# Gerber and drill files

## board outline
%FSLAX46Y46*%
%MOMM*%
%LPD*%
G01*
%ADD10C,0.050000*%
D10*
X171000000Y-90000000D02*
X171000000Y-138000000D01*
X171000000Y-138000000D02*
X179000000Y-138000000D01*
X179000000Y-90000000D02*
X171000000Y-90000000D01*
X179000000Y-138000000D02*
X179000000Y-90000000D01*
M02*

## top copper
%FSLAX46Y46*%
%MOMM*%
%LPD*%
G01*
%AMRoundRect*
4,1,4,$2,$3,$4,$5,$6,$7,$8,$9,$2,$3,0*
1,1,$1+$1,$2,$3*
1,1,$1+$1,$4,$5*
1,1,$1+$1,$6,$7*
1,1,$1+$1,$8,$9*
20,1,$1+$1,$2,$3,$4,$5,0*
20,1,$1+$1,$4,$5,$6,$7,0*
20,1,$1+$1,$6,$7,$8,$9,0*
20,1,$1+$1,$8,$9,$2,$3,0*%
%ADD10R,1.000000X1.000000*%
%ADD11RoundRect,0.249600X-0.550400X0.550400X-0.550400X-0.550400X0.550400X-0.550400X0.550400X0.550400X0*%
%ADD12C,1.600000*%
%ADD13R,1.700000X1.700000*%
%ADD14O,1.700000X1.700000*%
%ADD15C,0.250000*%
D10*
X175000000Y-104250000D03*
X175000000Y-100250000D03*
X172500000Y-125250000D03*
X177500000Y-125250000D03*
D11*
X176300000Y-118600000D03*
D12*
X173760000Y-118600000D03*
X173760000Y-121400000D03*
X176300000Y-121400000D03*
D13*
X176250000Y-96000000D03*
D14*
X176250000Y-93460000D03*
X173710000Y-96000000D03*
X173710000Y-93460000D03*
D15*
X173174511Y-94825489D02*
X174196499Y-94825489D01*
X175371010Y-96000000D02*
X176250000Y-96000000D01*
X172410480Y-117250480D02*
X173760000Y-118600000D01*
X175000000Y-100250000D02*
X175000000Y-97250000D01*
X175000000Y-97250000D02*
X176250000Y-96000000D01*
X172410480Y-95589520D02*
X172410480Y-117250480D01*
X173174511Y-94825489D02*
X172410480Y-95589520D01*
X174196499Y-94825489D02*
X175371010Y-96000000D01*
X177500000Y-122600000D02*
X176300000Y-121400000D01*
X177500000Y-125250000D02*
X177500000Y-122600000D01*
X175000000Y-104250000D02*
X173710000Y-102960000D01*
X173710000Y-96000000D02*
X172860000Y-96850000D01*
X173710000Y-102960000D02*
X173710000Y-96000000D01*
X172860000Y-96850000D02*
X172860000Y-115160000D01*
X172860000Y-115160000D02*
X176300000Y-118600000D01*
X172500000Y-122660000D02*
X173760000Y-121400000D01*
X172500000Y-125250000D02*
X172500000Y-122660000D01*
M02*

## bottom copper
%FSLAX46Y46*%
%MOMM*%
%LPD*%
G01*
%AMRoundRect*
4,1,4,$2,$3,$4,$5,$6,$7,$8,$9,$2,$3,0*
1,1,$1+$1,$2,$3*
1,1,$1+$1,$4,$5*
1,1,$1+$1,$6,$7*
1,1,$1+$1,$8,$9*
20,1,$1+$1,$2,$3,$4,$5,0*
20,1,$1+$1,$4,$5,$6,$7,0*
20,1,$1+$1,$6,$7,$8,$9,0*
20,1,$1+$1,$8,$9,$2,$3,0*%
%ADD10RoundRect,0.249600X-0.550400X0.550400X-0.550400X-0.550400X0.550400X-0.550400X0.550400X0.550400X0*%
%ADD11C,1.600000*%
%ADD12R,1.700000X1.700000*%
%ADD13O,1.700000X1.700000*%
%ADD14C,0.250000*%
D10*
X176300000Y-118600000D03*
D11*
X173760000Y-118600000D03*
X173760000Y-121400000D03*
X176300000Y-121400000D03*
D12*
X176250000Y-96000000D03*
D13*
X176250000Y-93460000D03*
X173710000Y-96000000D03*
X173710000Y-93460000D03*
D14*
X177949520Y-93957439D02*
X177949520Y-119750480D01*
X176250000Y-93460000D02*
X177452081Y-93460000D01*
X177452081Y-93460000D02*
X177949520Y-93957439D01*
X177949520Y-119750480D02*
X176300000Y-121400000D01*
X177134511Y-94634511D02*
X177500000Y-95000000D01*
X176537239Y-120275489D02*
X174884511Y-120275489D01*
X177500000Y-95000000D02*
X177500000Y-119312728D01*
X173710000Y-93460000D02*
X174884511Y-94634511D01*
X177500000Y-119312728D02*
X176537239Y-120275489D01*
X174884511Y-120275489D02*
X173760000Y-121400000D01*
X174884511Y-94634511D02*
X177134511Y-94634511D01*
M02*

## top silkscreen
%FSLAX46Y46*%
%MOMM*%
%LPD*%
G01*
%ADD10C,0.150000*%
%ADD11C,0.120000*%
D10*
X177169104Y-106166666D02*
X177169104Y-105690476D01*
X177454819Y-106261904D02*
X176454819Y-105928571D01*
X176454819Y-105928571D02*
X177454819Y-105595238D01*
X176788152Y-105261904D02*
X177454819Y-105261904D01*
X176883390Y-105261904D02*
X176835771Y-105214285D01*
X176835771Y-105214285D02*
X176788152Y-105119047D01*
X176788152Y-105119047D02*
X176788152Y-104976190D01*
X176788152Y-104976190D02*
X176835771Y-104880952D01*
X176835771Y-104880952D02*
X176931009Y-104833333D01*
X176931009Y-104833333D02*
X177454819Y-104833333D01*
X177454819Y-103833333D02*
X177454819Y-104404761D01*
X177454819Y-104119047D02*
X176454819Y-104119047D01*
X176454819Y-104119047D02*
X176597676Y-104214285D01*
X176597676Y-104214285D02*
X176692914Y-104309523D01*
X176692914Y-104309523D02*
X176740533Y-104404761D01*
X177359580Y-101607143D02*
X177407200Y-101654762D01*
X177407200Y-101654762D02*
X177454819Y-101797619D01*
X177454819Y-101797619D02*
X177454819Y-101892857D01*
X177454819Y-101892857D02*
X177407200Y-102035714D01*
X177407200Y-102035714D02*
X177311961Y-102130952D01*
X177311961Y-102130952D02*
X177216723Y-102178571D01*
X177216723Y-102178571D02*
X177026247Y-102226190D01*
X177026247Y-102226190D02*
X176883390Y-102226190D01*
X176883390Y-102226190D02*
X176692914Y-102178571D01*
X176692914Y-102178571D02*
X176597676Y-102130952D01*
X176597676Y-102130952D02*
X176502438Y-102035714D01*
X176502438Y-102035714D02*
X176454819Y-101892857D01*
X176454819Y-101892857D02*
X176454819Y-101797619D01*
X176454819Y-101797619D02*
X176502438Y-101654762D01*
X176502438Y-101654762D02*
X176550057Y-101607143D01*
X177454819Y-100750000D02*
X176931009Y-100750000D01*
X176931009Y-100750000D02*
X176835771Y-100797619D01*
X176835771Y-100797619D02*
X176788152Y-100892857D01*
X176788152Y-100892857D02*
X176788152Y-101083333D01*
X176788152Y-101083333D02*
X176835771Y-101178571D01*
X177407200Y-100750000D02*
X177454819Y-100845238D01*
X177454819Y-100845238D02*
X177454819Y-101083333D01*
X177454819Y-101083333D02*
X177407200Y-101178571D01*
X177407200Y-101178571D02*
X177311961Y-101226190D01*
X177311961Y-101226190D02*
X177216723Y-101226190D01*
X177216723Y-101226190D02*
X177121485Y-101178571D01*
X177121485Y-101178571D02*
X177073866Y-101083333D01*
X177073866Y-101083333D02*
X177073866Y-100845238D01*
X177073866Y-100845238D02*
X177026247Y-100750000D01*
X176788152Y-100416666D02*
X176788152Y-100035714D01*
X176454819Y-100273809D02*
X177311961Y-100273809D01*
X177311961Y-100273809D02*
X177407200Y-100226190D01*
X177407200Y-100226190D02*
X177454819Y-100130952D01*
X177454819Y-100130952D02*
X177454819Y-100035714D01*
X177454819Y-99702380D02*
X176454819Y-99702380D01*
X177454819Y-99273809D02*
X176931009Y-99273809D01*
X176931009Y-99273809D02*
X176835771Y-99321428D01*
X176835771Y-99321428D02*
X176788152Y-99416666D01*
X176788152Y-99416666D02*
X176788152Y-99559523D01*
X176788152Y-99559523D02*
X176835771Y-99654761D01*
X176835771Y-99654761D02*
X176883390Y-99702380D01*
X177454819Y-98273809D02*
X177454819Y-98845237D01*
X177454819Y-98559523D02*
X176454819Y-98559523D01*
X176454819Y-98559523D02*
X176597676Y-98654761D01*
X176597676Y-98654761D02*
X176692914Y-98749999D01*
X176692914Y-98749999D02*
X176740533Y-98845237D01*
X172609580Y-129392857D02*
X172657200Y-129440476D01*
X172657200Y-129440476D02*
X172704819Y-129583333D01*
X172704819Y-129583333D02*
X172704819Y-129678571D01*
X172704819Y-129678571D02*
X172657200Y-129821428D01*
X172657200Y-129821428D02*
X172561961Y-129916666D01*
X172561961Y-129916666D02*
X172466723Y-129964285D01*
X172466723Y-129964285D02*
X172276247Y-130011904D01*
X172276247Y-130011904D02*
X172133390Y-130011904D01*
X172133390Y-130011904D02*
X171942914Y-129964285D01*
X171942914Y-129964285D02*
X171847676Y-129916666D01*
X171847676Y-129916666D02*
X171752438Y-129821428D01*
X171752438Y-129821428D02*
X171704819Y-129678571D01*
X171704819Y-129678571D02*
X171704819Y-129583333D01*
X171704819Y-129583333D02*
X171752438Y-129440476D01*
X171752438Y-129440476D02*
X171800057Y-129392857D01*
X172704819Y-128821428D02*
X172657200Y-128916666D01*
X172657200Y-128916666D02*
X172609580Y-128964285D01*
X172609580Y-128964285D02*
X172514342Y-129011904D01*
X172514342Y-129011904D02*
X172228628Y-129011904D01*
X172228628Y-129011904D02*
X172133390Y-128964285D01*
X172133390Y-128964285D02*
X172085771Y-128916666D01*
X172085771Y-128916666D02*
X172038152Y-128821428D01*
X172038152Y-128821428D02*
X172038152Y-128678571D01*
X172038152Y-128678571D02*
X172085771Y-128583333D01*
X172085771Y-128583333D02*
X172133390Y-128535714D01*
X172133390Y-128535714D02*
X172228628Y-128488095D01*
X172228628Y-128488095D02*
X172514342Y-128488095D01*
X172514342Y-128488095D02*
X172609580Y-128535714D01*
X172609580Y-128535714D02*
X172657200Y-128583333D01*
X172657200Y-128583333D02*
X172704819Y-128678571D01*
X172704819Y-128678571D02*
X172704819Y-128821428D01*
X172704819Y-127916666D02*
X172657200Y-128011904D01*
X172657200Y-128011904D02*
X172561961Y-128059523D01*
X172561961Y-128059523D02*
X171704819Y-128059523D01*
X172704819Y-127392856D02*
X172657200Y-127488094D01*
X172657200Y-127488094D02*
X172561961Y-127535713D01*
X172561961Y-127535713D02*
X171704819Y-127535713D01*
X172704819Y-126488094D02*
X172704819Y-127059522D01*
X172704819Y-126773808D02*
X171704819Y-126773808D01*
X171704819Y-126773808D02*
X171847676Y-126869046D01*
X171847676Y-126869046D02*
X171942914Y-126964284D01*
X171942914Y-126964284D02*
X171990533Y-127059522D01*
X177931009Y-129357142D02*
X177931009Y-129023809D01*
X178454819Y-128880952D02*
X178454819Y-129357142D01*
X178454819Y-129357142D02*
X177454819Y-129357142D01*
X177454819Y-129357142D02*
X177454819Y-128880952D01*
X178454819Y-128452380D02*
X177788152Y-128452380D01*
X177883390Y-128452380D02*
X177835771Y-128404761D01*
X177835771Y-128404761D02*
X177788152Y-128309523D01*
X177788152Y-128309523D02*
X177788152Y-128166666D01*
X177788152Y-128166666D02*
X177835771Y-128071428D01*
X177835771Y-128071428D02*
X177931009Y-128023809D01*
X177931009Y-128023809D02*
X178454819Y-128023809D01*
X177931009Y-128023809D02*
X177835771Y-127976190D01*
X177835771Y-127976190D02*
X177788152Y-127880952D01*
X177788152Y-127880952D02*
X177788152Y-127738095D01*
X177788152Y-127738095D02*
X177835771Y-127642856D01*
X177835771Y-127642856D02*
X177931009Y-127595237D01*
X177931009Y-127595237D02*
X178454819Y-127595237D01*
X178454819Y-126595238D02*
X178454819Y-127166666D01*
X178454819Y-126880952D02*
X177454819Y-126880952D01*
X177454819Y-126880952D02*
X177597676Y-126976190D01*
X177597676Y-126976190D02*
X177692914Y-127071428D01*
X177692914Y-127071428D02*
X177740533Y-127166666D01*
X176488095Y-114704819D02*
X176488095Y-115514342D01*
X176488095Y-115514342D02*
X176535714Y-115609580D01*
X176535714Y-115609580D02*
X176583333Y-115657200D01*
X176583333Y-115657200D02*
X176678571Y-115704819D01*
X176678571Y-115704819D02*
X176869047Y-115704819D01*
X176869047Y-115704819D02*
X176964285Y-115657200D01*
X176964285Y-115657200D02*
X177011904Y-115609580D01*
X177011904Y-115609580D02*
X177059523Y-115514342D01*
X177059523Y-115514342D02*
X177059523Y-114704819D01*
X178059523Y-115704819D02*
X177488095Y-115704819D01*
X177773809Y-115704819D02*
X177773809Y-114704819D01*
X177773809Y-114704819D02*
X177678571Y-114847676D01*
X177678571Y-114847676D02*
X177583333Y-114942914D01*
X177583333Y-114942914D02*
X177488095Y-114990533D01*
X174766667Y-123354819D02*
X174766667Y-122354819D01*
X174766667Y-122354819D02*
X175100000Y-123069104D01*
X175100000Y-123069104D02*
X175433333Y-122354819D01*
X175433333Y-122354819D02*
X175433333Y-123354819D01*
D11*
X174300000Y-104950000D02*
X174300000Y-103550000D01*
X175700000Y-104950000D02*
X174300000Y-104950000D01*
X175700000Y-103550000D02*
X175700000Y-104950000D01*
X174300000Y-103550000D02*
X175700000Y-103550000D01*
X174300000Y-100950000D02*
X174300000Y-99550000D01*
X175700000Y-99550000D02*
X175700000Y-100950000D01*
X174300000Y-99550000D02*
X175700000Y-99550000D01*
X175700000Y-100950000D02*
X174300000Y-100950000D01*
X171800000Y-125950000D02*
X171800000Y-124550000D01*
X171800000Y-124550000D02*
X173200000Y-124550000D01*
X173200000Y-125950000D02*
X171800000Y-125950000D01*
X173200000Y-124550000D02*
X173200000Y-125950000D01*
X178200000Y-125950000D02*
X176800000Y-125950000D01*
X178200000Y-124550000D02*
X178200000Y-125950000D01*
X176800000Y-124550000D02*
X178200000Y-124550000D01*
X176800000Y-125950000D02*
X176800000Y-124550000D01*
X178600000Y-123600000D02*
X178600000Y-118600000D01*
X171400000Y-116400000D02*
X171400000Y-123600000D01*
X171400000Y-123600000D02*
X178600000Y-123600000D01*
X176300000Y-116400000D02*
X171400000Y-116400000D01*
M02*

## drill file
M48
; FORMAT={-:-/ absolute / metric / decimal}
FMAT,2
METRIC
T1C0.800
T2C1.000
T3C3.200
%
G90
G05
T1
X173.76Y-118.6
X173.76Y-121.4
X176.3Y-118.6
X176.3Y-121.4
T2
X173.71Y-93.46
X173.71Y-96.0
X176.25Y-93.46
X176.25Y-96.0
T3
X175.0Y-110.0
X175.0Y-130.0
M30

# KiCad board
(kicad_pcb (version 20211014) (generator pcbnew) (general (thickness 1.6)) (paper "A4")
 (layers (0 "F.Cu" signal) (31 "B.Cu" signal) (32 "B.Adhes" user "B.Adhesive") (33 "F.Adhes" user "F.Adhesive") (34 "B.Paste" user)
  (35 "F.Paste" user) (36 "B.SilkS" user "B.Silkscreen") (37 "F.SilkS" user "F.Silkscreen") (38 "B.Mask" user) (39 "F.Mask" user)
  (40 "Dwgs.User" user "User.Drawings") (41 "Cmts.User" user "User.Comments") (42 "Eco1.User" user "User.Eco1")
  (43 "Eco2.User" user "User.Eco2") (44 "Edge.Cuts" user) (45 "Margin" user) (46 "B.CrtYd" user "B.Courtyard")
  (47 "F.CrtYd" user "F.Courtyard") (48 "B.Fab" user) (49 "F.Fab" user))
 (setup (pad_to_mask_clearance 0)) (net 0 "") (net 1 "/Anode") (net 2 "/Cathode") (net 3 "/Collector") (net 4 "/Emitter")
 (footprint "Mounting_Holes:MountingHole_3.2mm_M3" (layer "F.Cu") (at 175 130)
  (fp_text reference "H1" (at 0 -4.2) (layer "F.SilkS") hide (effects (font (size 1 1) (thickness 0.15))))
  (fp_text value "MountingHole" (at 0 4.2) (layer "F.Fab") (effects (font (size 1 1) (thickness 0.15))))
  (pad "" np_thru_hole circle locked (at 0 0) (size 3.2 3.2) (drill 3.2) (layers *.Cu *.Mask)))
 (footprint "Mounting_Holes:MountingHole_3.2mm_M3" (layer "F.Cu") (at 175 110)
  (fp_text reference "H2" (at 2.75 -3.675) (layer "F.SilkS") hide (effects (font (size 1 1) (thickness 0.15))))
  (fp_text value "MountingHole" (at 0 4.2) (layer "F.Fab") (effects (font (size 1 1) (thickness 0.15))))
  (pad "" np_thru_hole circle locked (at 0 0) (size 3.2 3.2) (drill 3.2) (layers *.Cu *.Mask)))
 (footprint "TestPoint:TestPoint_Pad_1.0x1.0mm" (layer "F.Cu") (at 175 104.25)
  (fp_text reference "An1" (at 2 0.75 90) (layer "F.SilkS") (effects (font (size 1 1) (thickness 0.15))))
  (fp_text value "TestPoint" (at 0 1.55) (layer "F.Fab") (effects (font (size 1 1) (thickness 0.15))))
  (fp_line (start -0.7 0.7) (end -0.7 -0.7) (layer "F.SilkS") (width 0.12))
  (fp_line (start 0.7 0.7) (end -0.7 0.7) (layer "F.SilkS") (width 0.12))
  (fp_line (start 0.7 -0.7) (end 0.7 0.7) (layer "F.SilkS") (width 0.12))
  (fp_line (start -0.7 -0.7) (end 0.7 -0.7) (layer "F.SilkS") (width 0.12))
  (pad "1" smd rect locked (at 0 0) (size 1 1) (layers "F.Cu" "F.Mask") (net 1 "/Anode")))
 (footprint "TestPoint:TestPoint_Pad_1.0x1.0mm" (layer "F.Cu") (at 175 100.25)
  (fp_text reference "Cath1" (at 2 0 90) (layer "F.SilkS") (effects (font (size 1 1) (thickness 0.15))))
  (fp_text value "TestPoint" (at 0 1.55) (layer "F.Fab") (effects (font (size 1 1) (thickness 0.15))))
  (fp_line (start -0.7 0.7) (end -0.7 -0.7) (layer "F.SilkS") (width 0.12))
  (fp_line (start 0.7 -0.7) (end 0.7 0.7) (layer "F.SilkS") (width 0.12))
  (fp_line (start -0.7 -0.7) (end 0.7 -0.7) (layer "F.SilkS") (width 0.12))
  (fp_line (start 0.7 0.7) (end -0.7 0.7) (layer "F.SilkS") (width 0.12))
  (pad "1" smd rect locked (at 0 0) (size 1 1) (layers "F.Cu" "F.Mask") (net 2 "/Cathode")))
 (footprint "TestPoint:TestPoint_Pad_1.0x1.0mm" (layer "F.Cu") (at 172.5 125.25)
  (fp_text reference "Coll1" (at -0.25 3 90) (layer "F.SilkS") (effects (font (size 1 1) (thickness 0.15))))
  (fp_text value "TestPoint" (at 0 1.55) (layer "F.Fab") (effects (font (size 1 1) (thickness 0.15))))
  (fp_line (start -0.7 0.7) (end -0.7 -0.7) (layer "F.SilkS") (width 0.12))
  (fp_line (start -0.7 -0.7) (end 0.7 -0.7) (layer "F.SilkS") (width 0.12))
  (fp_line (start 0.7 0.7) (end -0.7 0.7) (layer "F.SilkS") (width 0.12))
  (fp_line (start 0.7 -0.7) (end 0.7 0.7) (layer "F.SilkS") (width 0.12))
  (pad "1" smd rect locked (at 0 0) (size 1 1) (layers "F.Cu" "F.Mask") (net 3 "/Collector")))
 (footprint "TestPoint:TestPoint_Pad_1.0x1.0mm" (layer "F.Cu") (at 177.5 125.25)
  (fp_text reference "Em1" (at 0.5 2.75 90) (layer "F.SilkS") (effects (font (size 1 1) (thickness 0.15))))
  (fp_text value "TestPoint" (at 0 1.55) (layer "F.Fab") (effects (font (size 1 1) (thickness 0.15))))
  (fp_line (start 0.7 0.7) (end -0.7 0.7) (layer "F.SilkS") (width 0.12))
  (fp_line (start 0.7 -0.7) (end 0.7 0.7) (layer "F.SilkS") (width 0.12))
  (fp_line (start -0.7 -0.7) (end 0.7 -0.7) (layer "F.SilkS") (width 0.12))
  (fp_line (start -0.7 0.7) (end -0.7 -0.7) (layer "F.SilkS") (width 0.12))
  (pad "1" smd rect locked (at 0 0) (size 1 1) (layers "F.Cu" "F.Mask") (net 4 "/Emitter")))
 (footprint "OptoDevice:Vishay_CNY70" (layer "F.Cu") (at 176.3 118.6 -90)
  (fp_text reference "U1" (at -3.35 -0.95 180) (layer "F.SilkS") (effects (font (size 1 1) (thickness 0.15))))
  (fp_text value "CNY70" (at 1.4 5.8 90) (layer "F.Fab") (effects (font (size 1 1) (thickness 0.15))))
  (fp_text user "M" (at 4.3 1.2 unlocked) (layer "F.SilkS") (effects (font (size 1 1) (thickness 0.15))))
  (fp_line (start 5 -2.3) (end 0 -2.3) (layer "F.SilkS") (width 0.12))
  (fp_line (start -2.2 4.9) (end 5 4.9) (layer "F.SilkS") (width 0.12))
  (fp_line (start 5 4.9) (end 5 -2.3) (layer "F.SilkS") (width 0.12))
  (fp_line (start -2.2 0) (end -2.2 4.9) (layer "F.SilkS") (width 0.12))
  (pad "1" thru_hole roundrect (at 0 0 270) (size 1.6 1.6) (drill 0.8) (layers *.Cu *.Mask) (roundrect_rratio 0.156) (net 1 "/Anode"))
  (pad "2" thru_hole circle (at 0 2.54 270) (size 1.6 1.6) (drill 0.8) (layers *.Cu *.Mask) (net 2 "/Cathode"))
  (pad "3" thru_hole circle (at 2.8 2.54 270) (size 1.6 1.6) (drill 0.8) (layers *.Cu *.Mask) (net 3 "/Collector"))
  (pad "4" thru_hole circle (at 2.8 0 270) (size 1.6 1.6) (drill 0.8) (layers *.Cu *.Mask) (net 4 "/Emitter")))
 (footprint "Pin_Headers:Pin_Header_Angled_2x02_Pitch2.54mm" (layer "B.Cu") (at 176.25 96 90)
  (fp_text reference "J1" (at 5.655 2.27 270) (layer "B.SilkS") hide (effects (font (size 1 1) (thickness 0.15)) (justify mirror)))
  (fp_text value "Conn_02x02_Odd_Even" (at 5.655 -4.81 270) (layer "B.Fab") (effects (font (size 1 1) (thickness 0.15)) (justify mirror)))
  (pad "1" thru_hole rect (at 0 0 90) (size 1.7 1.7) (drill 1) (layers *.Cu *.Mask) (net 2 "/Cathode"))
  (pad "2" thru_hole oval (at 2.54 0 90) (size 1.7 1.7) (drill 1) (layers *.Cu *.Mask) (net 4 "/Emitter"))
  (pad "3" thru_hole oval (at 0 -2.54 90) (size 1.7 1.7) (drill 1) (layers *.Cu *.Mask) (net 1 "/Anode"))
  (pad "4" thru_hole oval (at 2.54 -2.54 90) (size 1.7 1.7) (drill 1) (layers *.Cu *.Mask) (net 3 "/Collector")))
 (gr_line (start 171 90) (end 171 138) (layer "Edge.Cuts") (width 0.05))
 (gr_line (start 171 138) (end 179 138) (layer "Edge.Cuts") (width 0.05))
 (gr_line (start 179 90) (end 171 90) (layer "Edge.Cuts") (width 0.05))
 (gr_line (start 179 138) (end 179 90) (layer "Edge.Cuts") (width 0.05))
 (segment (start 173.174511 94.825489) (end 174.196499 94.825489) (width 0.25) (layer "F.Cu") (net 2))
 (segment (start 175.37101 96) (end 176.25 96) (width 0.25) (layer "F.Cu") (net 2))
 (segment (start 172.41048 117.25048) (end 173.76 118.6) (width 0.25) (layer "F.Cu") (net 2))
 (segment (start 175 100.25) (end 175 97.25) (width 0.25) (layer "F.Cu") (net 2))
 (segment (start 175 97.25) (end 176.25 96) (width 0.25) (layer "F.Cu") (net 2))
 (segment (start 172.41048 95.58952) (end 172.41048 117.25048) (width 0.25) (layer "F.Cu") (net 2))
 (segment (start 173.174511 94.825489) (end 172.41048 95.58952) (width 0.25) (layer "F.Cu") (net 2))
 (segment (start 174.196499 94.825489) (end 175.37101 96) (width 0.25) (layer "F.Cu") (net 2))
 (segment (start 177.5 122.6) (end 176.3 121.4) (width 0.25) (layer "F.Cu") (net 4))
 (segment (start 177.5 125.25) (end 177.5 122.6) (width 0.25) (layer "F.Cu") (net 4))
 (segment (start 177.94952 93.957439) (end 177.94952 119.75048) (width 0.25) (layer "B.Cu") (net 4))
 (segment (start 176.25 93.46) (end 177.452081 93.46) (width 0.25) (layer "B.Cu") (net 4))
 (segment (start 177.452081 93.46) (end 177.94952 93.957439) (width 0.25) (layer "B.Cu") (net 4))
 (segment (start 177.94952 119.75048) (end 176.3 121.4) (width 0.25) (layer "B.Cu") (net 4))
 (segment (start 175 104.25) (end 173.71 102.96) (width 0.25) (layer "F.Cu") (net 1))
 (segment (start 173.71 96) (end 172.86 96.85) (width 0.25) (layer "F.Cu") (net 1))
 (segment (start 173.71 102.96) (end 173.71 96) (width 0.25) (layer "F.Cu") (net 1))
 (segment (start 172.86 96.85) (end 172.86 115.16) (width 0.25) (layer "F.Cu") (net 1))
 (segment (start 172.86 115.16) (end 176.3 118.6) (width 0.25) (layer "F.Cu") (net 1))
 (segment (start 172.5 122.66) (end 173.76 121.4) (width 0.25) (layer "F.Cu") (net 3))
 (segment (start 172.5 125.25) (end 172.5 122.66) (width 0.25) (layer "F.Cu") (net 3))
 (segment (start 177.134511 94.634511) (end 177.5 95) (width 0.25) (layer "B.Cu") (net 3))
 (segment (start 176.537239 120.275489) (end 174.884511 120.275489) (width 0.25) (layer "B.Cu") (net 3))
 (segment (start 177.5 95) (end 177.5 119.312728) (width 0.25) (layer "B.Cu") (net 3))
 (segment (start 173.71 93.46) (end 174.884511 94.634511) (width 0.25) (layer "B.Cu") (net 3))
 (segment (start 177.5 119.312728) (end 176.537239 120.275489) (width 0.25) (layer "B.Cu") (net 3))
 (segment (start 174.884511 120.275489) (end 173.76 121.4) (width 0.25) (layer "B.Cu") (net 3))
 (segment (start 174.884511 94.634511) (end 177.134511 94.634511) (width 0.25) (layer "B.Cu") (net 3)))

